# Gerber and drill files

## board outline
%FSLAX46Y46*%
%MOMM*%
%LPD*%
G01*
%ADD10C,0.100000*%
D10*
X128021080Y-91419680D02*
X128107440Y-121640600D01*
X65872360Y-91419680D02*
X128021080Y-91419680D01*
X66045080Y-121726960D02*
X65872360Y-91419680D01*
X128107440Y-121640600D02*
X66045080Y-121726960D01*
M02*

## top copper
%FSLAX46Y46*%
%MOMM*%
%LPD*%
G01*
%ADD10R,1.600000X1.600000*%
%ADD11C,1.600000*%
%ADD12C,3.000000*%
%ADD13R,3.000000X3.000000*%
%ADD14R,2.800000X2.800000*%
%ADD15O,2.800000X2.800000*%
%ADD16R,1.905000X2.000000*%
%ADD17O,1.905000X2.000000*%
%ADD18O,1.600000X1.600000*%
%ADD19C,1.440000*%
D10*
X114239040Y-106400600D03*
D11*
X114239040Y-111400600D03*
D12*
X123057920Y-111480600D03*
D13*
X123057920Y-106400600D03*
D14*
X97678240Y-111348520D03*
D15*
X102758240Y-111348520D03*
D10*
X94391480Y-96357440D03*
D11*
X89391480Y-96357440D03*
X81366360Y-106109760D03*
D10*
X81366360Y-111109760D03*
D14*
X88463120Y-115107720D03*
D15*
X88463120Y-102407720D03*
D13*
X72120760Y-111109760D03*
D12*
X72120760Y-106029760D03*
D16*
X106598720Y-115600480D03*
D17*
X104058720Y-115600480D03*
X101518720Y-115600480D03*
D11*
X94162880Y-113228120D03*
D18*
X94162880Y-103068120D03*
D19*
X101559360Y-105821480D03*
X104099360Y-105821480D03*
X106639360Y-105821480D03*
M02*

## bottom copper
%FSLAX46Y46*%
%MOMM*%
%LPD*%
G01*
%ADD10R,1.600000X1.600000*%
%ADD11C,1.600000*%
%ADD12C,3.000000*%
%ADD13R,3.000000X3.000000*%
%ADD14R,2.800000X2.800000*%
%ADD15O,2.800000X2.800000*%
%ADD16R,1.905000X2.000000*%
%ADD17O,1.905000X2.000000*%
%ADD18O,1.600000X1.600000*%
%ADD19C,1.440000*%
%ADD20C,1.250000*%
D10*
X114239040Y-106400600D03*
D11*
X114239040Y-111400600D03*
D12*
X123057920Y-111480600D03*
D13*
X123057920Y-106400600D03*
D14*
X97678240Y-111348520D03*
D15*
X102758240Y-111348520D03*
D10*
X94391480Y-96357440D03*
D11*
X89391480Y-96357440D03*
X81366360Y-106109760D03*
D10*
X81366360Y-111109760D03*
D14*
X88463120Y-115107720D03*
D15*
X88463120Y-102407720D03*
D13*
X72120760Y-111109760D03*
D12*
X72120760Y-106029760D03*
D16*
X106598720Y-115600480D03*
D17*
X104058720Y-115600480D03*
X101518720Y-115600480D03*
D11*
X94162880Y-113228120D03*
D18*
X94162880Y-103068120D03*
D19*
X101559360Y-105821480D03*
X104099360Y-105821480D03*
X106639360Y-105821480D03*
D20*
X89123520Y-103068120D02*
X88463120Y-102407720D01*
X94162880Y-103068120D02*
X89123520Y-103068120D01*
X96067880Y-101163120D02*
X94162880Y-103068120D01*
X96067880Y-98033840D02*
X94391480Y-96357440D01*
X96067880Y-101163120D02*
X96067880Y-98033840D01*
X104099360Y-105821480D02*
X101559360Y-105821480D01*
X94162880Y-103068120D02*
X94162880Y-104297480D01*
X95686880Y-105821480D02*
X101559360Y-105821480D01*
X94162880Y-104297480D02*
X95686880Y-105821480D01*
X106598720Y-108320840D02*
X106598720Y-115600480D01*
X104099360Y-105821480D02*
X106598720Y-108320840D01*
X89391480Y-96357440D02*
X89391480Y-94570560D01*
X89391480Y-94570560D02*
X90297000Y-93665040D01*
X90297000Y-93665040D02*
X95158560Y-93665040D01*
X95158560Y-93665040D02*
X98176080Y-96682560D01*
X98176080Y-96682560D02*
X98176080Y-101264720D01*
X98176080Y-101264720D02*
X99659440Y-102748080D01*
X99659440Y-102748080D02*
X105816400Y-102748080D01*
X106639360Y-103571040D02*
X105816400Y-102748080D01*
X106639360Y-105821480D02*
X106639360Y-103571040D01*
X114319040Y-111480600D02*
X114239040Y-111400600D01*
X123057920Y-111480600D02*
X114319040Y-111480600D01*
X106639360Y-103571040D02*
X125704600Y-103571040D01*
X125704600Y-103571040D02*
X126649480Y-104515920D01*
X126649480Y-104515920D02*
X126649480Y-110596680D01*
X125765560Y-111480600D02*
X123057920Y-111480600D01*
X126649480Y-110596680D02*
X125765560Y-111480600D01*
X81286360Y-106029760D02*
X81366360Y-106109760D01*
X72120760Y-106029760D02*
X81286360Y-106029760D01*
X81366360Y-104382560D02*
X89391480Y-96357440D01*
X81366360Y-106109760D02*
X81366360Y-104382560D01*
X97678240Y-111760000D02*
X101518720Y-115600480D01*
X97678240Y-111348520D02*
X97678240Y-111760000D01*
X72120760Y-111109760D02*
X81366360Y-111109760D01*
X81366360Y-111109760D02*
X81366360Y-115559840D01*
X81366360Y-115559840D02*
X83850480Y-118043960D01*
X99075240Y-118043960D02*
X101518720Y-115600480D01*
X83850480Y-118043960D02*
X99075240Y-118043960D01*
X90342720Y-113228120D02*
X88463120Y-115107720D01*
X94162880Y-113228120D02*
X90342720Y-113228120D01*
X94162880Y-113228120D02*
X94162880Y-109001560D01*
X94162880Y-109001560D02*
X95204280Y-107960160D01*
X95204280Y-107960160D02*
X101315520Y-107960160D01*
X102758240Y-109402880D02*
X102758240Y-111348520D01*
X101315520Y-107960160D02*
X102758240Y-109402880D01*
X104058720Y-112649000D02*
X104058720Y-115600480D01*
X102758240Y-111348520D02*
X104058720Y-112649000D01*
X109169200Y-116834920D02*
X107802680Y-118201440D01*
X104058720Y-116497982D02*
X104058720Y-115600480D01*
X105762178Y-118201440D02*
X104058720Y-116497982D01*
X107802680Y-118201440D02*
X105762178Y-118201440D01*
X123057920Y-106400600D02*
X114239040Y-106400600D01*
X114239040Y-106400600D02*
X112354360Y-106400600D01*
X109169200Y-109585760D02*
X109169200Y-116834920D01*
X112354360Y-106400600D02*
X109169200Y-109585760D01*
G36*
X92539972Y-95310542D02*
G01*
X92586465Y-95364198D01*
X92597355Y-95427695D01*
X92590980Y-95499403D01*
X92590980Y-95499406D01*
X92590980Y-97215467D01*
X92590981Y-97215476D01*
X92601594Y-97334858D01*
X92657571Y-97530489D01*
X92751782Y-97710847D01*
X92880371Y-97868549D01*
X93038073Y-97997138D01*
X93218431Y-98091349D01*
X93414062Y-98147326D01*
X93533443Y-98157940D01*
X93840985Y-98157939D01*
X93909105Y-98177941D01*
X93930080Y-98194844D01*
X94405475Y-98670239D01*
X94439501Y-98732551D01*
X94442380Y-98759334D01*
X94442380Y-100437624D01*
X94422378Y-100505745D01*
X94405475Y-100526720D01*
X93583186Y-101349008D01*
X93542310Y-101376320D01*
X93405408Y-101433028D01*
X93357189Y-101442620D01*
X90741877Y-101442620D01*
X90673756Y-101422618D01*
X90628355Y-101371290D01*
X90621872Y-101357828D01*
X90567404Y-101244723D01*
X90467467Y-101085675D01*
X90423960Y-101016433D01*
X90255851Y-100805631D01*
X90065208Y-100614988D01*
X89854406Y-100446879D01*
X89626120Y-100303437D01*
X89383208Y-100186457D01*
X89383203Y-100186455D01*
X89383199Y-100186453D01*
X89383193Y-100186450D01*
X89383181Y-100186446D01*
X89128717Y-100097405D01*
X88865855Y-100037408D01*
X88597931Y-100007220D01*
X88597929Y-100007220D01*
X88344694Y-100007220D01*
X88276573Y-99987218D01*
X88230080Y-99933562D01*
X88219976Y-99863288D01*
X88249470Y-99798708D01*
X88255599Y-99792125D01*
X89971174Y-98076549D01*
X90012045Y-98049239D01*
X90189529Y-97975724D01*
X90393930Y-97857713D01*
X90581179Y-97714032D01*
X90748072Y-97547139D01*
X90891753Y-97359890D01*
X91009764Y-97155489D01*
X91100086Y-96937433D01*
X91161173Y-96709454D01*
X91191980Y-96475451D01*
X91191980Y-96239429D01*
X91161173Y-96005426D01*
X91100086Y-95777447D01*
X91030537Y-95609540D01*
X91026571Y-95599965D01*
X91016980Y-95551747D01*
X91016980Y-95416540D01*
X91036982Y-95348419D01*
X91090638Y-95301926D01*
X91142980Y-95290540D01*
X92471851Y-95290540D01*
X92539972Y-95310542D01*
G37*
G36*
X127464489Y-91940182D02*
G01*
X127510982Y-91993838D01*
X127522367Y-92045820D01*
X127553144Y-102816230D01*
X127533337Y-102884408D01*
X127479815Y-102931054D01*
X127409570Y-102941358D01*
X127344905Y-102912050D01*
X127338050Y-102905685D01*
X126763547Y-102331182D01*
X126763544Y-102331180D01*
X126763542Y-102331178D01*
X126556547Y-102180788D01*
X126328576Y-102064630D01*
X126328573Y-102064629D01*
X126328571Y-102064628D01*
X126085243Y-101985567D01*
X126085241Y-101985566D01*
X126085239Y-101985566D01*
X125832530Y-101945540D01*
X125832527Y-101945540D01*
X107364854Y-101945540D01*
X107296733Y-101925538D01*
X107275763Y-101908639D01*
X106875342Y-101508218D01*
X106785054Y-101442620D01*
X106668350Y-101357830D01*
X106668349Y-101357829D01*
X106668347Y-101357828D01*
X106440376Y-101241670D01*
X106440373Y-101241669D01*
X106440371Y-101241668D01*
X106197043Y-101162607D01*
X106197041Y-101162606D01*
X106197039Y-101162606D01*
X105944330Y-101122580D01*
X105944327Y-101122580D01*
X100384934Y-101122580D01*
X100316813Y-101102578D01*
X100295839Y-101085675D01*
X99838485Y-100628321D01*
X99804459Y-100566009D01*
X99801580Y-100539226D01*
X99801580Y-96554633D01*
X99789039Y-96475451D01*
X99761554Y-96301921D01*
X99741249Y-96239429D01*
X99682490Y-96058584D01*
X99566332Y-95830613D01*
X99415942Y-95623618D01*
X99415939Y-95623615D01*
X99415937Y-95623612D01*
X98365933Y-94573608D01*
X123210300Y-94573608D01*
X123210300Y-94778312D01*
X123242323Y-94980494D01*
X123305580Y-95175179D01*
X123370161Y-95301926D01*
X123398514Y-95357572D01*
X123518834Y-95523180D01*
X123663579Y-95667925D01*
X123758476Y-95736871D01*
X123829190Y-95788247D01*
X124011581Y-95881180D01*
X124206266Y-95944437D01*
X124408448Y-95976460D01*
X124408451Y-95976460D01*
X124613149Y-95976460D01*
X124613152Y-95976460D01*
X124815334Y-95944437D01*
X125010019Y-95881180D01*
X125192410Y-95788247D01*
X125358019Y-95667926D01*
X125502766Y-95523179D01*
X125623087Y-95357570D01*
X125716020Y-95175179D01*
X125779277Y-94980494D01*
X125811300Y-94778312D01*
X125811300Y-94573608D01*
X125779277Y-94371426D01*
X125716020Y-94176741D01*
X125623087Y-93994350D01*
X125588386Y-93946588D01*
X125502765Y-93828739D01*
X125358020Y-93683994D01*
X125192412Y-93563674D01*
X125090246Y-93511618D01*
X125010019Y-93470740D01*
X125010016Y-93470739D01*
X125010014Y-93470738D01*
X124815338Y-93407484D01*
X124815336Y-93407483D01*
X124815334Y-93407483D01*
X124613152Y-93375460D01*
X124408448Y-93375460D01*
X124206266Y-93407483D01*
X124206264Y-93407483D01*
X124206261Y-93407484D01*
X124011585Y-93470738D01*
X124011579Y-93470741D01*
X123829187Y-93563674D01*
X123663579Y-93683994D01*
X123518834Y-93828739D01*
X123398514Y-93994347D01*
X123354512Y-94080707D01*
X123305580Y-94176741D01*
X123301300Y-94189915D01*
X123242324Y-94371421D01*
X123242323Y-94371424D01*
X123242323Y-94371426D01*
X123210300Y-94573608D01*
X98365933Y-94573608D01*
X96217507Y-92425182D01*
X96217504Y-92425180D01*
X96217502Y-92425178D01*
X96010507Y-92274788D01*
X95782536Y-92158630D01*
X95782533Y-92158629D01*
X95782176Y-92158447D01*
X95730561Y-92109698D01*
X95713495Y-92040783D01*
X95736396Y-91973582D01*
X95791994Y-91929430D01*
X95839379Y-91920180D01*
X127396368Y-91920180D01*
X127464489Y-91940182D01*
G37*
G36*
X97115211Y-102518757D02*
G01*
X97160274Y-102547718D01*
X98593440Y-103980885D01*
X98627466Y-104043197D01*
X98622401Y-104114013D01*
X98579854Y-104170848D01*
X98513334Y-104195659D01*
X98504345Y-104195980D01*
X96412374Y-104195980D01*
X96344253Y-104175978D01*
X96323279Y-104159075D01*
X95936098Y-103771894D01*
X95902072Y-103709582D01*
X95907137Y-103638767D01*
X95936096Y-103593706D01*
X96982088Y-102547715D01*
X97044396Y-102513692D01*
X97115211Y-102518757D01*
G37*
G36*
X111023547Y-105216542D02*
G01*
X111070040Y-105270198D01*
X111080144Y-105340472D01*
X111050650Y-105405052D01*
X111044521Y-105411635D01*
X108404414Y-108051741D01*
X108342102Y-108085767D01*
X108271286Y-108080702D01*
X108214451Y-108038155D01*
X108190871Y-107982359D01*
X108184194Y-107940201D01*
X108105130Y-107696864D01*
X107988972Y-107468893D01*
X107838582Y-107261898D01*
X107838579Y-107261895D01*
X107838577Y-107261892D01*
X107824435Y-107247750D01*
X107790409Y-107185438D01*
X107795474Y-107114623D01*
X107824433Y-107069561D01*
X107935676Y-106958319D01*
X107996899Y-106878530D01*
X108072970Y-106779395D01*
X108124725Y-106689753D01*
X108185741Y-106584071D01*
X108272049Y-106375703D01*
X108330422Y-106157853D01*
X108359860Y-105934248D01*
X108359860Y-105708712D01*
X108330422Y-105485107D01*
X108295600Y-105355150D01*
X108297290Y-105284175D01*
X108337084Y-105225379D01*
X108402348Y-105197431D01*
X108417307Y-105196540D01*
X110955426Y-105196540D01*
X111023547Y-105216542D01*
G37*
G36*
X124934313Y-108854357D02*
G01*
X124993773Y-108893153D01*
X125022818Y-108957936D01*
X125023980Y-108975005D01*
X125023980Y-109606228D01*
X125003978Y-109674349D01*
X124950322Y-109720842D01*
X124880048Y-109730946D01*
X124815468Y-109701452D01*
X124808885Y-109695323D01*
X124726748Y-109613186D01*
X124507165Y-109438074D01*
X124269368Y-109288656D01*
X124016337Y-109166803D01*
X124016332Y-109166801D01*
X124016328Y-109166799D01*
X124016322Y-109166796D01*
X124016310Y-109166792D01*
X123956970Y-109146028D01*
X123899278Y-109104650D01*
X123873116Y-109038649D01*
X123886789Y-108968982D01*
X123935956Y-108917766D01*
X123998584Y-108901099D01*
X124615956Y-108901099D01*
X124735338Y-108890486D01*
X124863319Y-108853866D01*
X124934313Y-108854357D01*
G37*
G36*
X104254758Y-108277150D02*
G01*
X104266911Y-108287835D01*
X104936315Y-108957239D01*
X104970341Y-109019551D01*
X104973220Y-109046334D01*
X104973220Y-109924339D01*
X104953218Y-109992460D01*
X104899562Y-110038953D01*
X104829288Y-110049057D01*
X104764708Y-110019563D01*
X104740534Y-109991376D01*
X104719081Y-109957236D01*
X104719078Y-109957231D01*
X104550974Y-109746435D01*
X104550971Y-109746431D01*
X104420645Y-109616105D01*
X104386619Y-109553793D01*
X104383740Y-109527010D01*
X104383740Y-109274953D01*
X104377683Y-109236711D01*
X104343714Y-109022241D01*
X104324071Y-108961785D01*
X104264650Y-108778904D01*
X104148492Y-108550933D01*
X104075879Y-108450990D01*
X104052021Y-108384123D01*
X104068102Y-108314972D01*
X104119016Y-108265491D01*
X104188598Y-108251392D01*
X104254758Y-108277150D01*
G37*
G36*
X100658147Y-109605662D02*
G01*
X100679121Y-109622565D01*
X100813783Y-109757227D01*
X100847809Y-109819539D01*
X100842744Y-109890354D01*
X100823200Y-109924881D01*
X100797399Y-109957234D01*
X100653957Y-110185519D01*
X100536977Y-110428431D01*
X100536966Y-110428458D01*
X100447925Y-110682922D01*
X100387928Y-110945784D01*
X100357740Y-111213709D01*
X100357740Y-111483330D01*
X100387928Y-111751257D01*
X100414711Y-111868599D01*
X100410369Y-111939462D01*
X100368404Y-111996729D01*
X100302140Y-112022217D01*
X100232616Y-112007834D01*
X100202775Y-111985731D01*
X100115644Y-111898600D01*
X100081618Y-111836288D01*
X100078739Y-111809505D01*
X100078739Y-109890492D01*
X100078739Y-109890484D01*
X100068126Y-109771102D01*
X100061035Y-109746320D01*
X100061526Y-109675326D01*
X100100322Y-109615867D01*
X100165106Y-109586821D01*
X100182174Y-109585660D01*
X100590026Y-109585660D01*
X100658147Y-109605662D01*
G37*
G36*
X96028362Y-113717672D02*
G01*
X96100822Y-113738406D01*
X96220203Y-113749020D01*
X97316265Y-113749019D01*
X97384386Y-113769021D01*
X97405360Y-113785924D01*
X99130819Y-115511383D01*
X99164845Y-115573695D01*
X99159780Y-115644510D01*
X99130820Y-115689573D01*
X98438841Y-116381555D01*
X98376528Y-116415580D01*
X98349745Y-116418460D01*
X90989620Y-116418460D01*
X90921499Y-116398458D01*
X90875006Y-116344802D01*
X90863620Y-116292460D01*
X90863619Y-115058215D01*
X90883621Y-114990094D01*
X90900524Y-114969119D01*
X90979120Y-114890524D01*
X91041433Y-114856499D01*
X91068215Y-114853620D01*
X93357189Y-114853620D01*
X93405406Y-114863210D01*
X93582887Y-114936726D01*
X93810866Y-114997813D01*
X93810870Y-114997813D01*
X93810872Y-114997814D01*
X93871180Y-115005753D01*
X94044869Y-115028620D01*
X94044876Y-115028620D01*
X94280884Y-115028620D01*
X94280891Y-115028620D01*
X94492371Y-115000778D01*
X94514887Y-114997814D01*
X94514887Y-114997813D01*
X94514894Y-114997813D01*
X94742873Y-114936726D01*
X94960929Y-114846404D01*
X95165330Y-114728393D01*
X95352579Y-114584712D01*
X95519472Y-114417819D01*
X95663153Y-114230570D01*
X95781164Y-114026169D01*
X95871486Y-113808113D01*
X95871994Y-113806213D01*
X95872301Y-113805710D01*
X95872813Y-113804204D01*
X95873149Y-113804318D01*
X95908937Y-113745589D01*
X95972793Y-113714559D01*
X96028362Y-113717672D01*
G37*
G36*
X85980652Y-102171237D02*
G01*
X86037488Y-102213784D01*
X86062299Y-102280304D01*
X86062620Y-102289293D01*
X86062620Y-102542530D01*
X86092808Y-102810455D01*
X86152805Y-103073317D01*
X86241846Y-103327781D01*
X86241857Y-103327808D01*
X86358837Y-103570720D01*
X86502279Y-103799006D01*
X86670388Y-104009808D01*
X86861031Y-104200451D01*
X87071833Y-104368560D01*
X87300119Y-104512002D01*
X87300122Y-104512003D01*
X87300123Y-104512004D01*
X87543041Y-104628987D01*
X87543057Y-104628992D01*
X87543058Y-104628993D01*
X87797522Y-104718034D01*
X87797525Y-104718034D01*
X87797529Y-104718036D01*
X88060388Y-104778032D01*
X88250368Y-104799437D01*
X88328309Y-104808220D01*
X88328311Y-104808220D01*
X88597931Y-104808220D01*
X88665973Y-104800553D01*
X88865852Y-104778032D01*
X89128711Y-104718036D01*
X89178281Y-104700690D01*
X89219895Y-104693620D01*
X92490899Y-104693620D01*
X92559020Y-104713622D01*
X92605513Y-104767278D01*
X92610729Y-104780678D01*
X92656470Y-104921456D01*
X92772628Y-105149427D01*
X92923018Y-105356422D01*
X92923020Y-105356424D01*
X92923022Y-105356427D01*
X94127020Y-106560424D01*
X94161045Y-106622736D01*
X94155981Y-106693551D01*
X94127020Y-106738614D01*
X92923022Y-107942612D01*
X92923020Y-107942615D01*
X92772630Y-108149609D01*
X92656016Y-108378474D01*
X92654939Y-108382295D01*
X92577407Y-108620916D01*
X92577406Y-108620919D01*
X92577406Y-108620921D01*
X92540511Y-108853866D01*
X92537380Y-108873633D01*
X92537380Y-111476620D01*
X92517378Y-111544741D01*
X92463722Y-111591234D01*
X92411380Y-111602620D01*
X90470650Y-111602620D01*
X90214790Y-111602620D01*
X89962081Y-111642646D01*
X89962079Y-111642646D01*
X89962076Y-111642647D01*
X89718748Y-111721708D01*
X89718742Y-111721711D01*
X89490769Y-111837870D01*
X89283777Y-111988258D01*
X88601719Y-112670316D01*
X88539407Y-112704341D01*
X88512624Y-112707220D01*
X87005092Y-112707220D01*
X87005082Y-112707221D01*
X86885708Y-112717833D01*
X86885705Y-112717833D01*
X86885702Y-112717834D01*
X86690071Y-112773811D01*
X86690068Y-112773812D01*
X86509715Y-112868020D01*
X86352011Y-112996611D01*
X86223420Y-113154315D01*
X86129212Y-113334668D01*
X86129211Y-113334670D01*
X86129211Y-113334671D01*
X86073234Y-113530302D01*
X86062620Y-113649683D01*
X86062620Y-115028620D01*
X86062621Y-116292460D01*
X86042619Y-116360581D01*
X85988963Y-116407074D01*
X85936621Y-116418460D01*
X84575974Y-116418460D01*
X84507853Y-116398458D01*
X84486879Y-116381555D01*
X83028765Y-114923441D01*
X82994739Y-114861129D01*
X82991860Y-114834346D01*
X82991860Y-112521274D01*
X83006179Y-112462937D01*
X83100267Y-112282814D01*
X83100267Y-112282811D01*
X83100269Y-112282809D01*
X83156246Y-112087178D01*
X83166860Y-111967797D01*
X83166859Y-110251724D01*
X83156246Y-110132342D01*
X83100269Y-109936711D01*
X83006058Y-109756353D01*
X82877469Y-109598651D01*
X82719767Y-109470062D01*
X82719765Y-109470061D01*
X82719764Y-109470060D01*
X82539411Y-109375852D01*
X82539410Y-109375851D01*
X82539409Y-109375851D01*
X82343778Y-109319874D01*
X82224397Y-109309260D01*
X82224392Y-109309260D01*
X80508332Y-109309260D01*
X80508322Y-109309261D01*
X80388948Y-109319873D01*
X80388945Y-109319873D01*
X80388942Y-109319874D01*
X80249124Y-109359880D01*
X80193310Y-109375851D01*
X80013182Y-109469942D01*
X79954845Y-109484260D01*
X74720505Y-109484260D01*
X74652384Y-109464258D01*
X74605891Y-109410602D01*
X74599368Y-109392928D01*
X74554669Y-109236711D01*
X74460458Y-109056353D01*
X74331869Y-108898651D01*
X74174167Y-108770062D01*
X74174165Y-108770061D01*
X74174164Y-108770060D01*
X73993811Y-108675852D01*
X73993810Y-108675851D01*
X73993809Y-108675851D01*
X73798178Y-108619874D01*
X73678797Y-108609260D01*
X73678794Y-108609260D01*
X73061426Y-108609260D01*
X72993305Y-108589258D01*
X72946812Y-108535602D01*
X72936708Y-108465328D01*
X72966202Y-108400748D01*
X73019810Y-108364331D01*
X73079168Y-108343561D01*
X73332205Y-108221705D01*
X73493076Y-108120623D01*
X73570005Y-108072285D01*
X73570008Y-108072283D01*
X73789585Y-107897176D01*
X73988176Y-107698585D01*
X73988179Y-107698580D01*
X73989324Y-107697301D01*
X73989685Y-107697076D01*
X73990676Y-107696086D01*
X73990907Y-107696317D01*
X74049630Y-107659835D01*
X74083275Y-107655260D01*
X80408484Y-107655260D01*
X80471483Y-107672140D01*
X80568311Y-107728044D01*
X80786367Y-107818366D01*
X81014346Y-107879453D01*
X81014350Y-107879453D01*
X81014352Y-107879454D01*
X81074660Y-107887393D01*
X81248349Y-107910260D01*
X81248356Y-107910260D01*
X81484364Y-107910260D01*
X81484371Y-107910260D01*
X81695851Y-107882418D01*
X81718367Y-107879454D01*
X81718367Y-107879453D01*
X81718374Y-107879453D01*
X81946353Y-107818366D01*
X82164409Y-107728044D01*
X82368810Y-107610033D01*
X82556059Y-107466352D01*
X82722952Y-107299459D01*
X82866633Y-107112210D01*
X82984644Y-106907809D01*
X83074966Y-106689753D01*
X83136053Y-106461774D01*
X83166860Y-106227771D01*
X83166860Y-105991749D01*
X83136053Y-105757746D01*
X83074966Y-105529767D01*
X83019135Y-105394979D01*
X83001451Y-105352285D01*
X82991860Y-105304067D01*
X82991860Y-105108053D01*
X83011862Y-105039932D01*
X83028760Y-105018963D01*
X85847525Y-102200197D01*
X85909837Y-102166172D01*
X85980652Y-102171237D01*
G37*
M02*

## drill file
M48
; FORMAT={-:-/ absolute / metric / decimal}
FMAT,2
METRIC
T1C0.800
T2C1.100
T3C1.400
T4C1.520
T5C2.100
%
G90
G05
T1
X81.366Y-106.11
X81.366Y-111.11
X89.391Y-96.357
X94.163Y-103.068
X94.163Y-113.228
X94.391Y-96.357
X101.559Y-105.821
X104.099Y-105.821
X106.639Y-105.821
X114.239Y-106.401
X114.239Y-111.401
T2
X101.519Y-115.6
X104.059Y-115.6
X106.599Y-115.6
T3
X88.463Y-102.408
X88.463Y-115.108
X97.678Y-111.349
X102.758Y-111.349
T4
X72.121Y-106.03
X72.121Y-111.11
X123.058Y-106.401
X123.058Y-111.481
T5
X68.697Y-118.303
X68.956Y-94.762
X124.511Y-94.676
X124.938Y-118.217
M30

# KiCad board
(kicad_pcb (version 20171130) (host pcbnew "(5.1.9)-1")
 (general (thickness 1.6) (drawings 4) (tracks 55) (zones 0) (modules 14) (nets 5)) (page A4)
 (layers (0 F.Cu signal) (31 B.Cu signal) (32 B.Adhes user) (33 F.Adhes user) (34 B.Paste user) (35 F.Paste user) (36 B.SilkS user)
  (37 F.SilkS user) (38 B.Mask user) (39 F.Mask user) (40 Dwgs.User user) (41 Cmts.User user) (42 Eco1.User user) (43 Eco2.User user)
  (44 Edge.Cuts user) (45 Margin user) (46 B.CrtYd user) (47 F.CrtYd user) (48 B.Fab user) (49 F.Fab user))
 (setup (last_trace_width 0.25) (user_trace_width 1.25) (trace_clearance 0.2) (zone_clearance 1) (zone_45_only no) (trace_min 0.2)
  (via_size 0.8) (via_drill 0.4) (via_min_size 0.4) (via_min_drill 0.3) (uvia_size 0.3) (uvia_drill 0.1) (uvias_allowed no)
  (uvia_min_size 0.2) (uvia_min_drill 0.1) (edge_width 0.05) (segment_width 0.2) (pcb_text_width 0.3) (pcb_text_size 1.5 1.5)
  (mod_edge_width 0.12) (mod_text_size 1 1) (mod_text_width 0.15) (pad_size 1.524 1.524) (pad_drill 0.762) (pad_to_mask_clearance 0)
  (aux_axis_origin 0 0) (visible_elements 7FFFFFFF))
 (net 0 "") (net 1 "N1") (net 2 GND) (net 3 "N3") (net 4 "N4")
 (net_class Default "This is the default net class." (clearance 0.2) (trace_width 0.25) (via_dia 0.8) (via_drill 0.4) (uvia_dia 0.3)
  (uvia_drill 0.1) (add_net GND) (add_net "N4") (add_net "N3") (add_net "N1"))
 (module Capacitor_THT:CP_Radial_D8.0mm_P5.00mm (layer F.Cu) (at 114.23904 106.4006 270)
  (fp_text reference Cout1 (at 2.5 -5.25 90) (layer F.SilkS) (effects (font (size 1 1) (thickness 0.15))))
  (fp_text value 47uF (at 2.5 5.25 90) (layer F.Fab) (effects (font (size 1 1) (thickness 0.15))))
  (pad 1 thru_hole rect (at 0 0 270) (size 1.6 1.6) (drill 0.8) (layers *.Cu *.Mask) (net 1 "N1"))
  (pad 2 thru_hole circle (at 5 0 270) (size 1.6 1.6) (drill 0.8) (layers *.Cu *.Mask) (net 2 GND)))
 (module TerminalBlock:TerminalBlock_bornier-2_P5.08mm (layer F.Cu) (at 123.05792 106.4006 270)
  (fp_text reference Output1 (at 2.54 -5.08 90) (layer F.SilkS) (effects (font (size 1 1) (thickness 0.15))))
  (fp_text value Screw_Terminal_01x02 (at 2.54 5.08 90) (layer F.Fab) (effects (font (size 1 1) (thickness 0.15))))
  (pad 2 thru_hole circle (at 5.08 0 270) (size 3 3) (drill 1.52) (layers *.Cu *.Mask) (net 2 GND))
  (pad 1 thru_hole rect (at 0 0 270) (size 3 3) (drill 1.52) (layers *.Cu *.Mask) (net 1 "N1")))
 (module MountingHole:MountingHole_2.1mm (layer F.Cu) (at 68.95592 94.76232)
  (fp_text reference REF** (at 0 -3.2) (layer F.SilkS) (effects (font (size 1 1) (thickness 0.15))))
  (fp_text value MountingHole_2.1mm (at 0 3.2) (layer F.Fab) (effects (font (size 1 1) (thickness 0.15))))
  (pad "" np_thru_hole circle (at 0 0) (size 2.1 2.1) (drill 2.1) (layers *.Cu *.Mask)))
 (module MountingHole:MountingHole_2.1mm (layer F.Cu) (at 68.69684 118.30304)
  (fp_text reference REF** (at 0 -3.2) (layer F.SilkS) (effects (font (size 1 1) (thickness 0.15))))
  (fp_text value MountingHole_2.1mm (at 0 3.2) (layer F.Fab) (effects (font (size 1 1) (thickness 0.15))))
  (pad "" np_thru_hole circle (at 0 0) (size 2.1 2.1) (drill 2.1) (layers *.Cu *.Mask)))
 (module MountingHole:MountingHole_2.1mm (layer F.Cu) (at 124.93752 118.21668)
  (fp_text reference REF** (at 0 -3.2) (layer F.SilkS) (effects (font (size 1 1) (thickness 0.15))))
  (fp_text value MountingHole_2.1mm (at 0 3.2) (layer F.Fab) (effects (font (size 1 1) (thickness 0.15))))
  (pad "" np_thru_hole circle (at 0 0) (size 2.1 2.1) (drill 2.1) (layers *.Cu *.Mask)))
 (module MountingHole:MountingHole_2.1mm (layer F.Cu) (at 124.5108 94.67596)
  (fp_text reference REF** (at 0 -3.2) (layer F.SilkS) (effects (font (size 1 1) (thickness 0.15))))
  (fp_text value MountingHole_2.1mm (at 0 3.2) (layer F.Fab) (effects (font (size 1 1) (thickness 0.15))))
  (pad "" np_thru_hole circle (at 0 0) (size 2.1 2.1) (drill 2.1) (layers *.Cu *.Mask)))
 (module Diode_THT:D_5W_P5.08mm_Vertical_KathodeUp (layer F.Cu) (at 97.67824 111.34852)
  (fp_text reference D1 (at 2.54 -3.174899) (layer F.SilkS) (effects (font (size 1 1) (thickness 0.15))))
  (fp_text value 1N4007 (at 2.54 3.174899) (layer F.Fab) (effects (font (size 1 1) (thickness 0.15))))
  (pad 1 thru_hole rect (at 0 0) (size 2.8 2.8) (drill 1.4) (layers *.Cu *.Mask) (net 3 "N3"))
  (pad 2 thru_hole oval (at 5.08 0) (size 2.8 2.8) (drill 1.4) (layers *.Cu *.Mask) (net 1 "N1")))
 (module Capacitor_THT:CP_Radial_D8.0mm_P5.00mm (layer F.Cu) (at 94.39148 96.35744 180)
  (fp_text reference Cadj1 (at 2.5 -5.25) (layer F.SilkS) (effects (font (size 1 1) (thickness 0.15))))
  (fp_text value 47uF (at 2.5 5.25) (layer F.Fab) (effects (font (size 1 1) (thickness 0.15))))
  (pad 1 thru_hole rect (at 0 0 180) (size 1.6 1.6) (drill 0.8) (layers *.Cu *.Mask) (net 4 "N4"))
  (pad 2 thru_hole circle (at 5 0 180) (size 1.6 1.6) (drill 0.8) (layers *.Cu *.Mask) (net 2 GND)))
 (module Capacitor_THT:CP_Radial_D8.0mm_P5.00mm (layer F.Cu) (at 81.36636 111.10976 90)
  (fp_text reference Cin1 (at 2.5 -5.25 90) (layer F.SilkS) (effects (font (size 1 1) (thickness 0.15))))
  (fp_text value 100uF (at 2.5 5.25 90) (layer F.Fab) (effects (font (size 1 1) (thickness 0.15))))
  (pad 2 thru_hole circle (at 5 0 90) (size 1.6 1.6) (drill 0.8) (layers *.Cu *.Mask) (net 2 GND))
  (pad 1 thru_hole rect (at 0 0 90) (size 1.6 1.6) (drill 0.8) (layers *.Cu *.Mask) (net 3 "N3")))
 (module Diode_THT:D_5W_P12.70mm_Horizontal (layer F.Cu) (at 88.46312 115.10772 90)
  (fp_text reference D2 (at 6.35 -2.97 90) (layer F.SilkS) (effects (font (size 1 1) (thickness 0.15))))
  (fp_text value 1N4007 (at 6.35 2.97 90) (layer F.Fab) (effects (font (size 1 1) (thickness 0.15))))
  (pad 1 thru_hole rect (at 0 0 90) (size 2.8 2.8) (drill 1.4) (layers *.Cu *.Mask) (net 1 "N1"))
  (pad 2 thru_hole oval (at 12.7 0 90) (size 2.8 2.8) (drill 1.4) (layers *.Cu *.Mask) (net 4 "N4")))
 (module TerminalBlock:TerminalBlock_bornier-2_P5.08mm (layer F.Cu) (at 72.12076 111.10976 90)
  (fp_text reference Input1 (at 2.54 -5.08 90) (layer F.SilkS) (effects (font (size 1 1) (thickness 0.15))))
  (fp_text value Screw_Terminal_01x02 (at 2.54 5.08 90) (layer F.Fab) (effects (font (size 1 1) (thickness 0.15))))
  (pad 1 thru_hole rect (at 0 0 90) (size 3 3) (drill 1.52) (layers *.Cu *.Mask) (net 3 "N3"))
  (pad 2 thru_hole circle (at 5.08 0 90) (size 3 3) (drill 1.52) (layers *.Cu *.Mask) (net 2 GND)))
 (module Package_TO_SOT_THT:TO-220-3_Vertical (layer F.Cu) (at 106.59872 115.60048 180)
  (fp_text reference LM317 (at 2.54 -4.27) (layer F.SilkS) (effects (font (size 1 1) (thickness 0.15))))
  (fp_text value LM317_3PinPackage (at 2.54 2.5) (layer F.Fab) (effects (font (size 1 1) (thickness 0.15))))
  (pad 1 thru_hole rect (at 0 0 180) (size 1.905 2) (drill 1.1) (layers *.Cu *.Mask) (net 4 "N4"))
  (pad 2 thru_hole oval (at 2.54 0 180) (size 1.905 2) (drill 1.1) (layers *.Cu *.Mask) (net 1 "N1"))
  (pad 3 thru_hole oval (at 5.08 0 180) (size 1.905 2) (drill 1.1) (layers *.Cu *.Mask) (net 3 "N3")))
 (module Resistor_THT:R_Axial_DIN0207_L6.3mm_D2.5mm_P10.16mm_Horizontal (layer F.Cu) (at 94.16288 113.22812 90)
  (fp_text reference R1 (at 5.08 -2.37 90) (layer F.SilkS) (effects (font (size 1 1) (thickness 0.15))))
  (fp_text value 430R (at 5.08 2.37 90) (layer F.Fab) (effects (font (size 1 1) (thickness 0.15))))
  (pad 1 thru_hole circle (at 0 0 90) (size 1.6 1.6) (drill 0.8) (layers *.Cu *.Mask) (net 1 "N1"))
  (pad 2 thru_hole oval (at 10.16 0 90) (size 1.6 1.6) (drill 0.8) (layers *.Cu *.Mask) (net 4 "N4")))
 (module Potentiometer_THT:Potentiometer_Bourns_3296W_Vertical (layer F.Cu) (at 101.55936 105.82148 180)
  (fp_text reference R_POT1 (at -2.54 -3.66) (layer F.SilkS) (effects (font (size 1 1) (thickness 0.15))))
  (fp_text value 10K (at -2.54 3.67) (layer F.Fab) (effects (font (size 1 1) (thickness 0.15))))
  (pad 1 thru_hole circle (at 0 0 180) (size 1.44 1.44) (drill 0.8) (layers *.Cu *.Mask) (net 4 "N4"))
  (pad 2 thru_hole circle (at -2.54 0 180) (size 1.44 1.44) (drill 0.8) (layers *.Cu *.Mask) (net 4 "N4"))
  (pad 3 thru_hole circle (at -5.08 0 180) (size 1.44 1.44) (drill 0.8) (layers *.Cu *.Mask) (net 2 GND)))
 (gr_line (start 128.02108 91.41968) (end 128.10744 121.6406) (layer Edge.Cuts) (width 0.1))
 (gr_line (start 65.87236 91.41968) (end 128.02108 91.41968) (layer Edge.Cuts) (width 0.1))
 (gr_line (start 66.04508 121.72696) (end 65.87236 91.41968) (layer Edge.Cuts) (width 0.1))
 (gr_line (start 128.10744 121.6406) (end 66.04508 121.72696) (layer Edge.Cuts) (width 0.1))
 (segment (start 89.12352 103.06812) (end 88.46312 102.40772) (width 1.25) (layer B.Cu) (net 4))
 (segment (start 94.16288 103.06812) (end 89.12352 103.06812) (width 1.25) (layer B.Cu) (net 4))
 (segment (start 96.06788 101.16312) (end 94.16288 103.06812) (width 1.25) (layer B.Cu) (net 4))
 (segment (start 96.06788 98.03384) (end 94.39148 96.35744) (width 1.25) (layer B.Cu) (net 4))
 (segment (start 96.06788 101.16312) (end 96.06788 98.03384) (width 1.25) (layer B.Cu) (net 4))
 (segment (start 104.09936 105.82148) (end 101.55936 105.82148) (width 1.25) (layer B.Cu) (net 4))
 (segment (start 94.16288 103.06812) (end 94.16288 104.29748) (width 1.25) (layer B.Cu) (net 4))
 (segment (start 95.68688 105.82148) (end 101.55936 105.82148) (width 1.25) (layer B.Cu) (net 4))
 (segment (start 94.16288 104.29748) (end 95.68688 105.82148) (width 1.25) (layer B.Cu) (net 4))
 (segment (start 106.59872 108.32084) (end 106.59872 115.60048) (width 1.25) (layer B.Cu) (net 4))
 (segment (start 104.09936 105.82148) (end 106.59872 108.32084) (width 1.25) (layer B.Cu) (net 4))
 (segment (start 89.39148 96.35744) (end 89.39148 94.57056) (width 1.25) (layer B.Cu) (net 2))
 (segment (start 89.39148 94.57056) (end 90.297 93.66504) (width 1.25) (layer B.Cu) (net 2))
 (segment (start 90.297 93.66504) (end 95.15856 93.66504) (width 1.25) (layer B.Cu) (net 2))
 (segment (start 95.15856 93.66504) (end 98.17608 96.68256) (width 1.25) (layer B.Cu) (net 2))
 (segment (start 98.17608 96.68256) (end 98.17608 101.26472) (width 1.25) (layer B.Cu) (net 2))
 (segment (start 98.17608 101.26472) (end 99.65944 102.74808) (width 1.25) (layer B.Cu) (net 2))
 (segment (start 99.65944 102.74808) (end 105.8164 102.74808) (width 1.25) (layer B.Cu) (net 2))
 (segment (start 106.63936 103.57104) (end 105.8164 102.74808) (width 1.25) (layer B.Cu) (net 2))
 (segment (start 106.63936 105.82148) (end 106.63936 103.57104) (width 1.25) (layer B.Cu) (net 2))
 (segment (start 114.31904 111.4806) (end 114.23904 111.4006) (width 1.25) (layer B.Cu) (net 2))
 (segment (start 123.05792 111.4806) (end 114.31904 111.4806) (width 1.25) (layer B.Cu) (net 2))
 (segment (start 106.63936 103.57104) (end 125.7046 103.57104) (width 1.25) (layer B.Cu) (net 2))
 (segment (start 125.7046 103.57104) (end 126.64948 104.51592) (width 1.25) (layer B.Cu) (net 2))
 (segment (start 126.64948 104.51592) (end 126.64948 110.59668) (width 1.25) (layer B.Cu) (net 2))
 (segment (start 125.76556 111.4806) (end 123.05792 111.4806) (width 1.25) (layer B.Cu) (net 2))
 (segment (start 126.64948 110.59668) (end 125.76556 111.4806) (width 1.25) (layer B.Cu) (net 2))
 (segment (start 81.28636 106.02976) (end 81.36636 106.10976) (width 1.25) (layer B.Cu) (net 2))
 (segment (start 72.12076 106.02976) (end 81.28636 106.02976) (width 1.25) (layer B.Cu) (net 2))
 (segment (start 81.36636 104.38256) (end 89.39148 96.35744) (width 1.25) (layer B.Cu) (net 2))
 (segment (start 81.36636 106.10976) (end 81.36636 104.38256) (width 1.25) (layer B.Cu) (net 2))
 (segment (start 97.67824 111.76) (end 101.51872 115.60048) (width 1.25) (layer B.Cu) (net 3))
 (segment (start 97.67824 111.34852) (end 97.67824 111.76) (width 1.25) (layer B.Cu) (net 3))
 (segment (start 72.12076 111.10976) (end 81.36636 111.10976) (width 1.25) (layer B.Cu) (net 3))
 (segment (start 81.36636 111.10976) (end 81.36636 115.55984) (width 1.25) (layer B.Cu) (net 3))
 (segment (start 81.36636 115.55984) (end 83.85048 118.04396) (width 1.25) (layer B.Cu) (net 3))
 (segment (start 99.07524 118.04396) (end 101.51872 115.60048) (width 1.25) (layer B.Cu) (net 3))
 (segment (start 83.85048 118.04396) (end 99.07524 118.04396) (width 1.25) (layer B.Cu) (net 3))
 (segment (start 90.34272 113.22812) (end 88.46312 115.10772) (width 1.25) (layer B.Cu) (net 1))
 (segment (start 94.16288 113.22812) (end 90.34272 113.22812) (width 1.25) (layer B.Cu) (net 1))
 (segment (start 94.16288 113.22812) (end 94.16288 109.00156) (width 1.25) (layer B.Cu) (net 1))
 (segment (start 94.16288 109.00156) (end 95.20428 107.96016) (width 1.25) (layer B.Cu) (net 1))
 (segment (start 95.20428 107.96016) (end 101.31552 107.96016) (width 1.25) (layer B.Cu) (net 1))
 (segment (start 102.75824 109.40288) (end 102.75824 111.34852) (width 1.25) (layer B.Cu) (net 1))
 (segment (start 101.31552 107.96016) (end 102.75824 109.40288) (width 1.25) (layer B.Cu) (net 1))
 (segment (start 104.05872 112.649) (end 104.05872 115.60048) (width 1.25) (layer B.Cu) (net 1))
 (segment (start 102.75824 111.34852) (end 104.05872 112.649) (width 1.25) (layer B.Cu) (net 1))
 (segment (start 109.1692 116.83492) (end 107.80268 118.20144) (width 1.25) (layer B.Cu) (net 1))
 (segment (start 104.05872 116.497982) (end 104.05872 115.60048) (width 1.25) (layer B.Cu) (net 1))
 (segment (start 105.762178 118.20144) (end 104.05872 116.497982) (width 1.25) (layer B.Cu) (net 1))
 (segment (start 107.80268 118.20144) (end 105.762178 118.20144) (width 1.25) (layer B.Cu) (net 1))
 (segment (start 123.05792 106.4006) (end 114.23904 106.4006) (width 1.25) (layer B.Cu) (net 1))
 (segment (start 114.23904 106.4006) (end 112.35436 106.4006) (width 1.25) (layer B.Cu) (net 1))
 (segment (start 109.1692 109.58576) (end 109.1692 116.83492) (width 1.25) (layer B.Cu) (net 1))
 (segment (start 112.35436 106.4006) (end 109.1692 109.58576) (width 1.25) (layer B.Cu) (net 1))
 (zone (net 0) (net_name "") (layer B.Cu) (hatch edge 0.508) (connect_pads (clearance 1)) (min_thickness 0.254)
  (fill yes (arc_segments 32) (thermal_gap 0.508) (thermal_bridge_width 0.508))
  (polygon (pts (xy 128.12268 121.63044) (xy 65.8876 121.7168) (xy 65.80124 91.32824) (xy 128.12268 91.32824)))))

